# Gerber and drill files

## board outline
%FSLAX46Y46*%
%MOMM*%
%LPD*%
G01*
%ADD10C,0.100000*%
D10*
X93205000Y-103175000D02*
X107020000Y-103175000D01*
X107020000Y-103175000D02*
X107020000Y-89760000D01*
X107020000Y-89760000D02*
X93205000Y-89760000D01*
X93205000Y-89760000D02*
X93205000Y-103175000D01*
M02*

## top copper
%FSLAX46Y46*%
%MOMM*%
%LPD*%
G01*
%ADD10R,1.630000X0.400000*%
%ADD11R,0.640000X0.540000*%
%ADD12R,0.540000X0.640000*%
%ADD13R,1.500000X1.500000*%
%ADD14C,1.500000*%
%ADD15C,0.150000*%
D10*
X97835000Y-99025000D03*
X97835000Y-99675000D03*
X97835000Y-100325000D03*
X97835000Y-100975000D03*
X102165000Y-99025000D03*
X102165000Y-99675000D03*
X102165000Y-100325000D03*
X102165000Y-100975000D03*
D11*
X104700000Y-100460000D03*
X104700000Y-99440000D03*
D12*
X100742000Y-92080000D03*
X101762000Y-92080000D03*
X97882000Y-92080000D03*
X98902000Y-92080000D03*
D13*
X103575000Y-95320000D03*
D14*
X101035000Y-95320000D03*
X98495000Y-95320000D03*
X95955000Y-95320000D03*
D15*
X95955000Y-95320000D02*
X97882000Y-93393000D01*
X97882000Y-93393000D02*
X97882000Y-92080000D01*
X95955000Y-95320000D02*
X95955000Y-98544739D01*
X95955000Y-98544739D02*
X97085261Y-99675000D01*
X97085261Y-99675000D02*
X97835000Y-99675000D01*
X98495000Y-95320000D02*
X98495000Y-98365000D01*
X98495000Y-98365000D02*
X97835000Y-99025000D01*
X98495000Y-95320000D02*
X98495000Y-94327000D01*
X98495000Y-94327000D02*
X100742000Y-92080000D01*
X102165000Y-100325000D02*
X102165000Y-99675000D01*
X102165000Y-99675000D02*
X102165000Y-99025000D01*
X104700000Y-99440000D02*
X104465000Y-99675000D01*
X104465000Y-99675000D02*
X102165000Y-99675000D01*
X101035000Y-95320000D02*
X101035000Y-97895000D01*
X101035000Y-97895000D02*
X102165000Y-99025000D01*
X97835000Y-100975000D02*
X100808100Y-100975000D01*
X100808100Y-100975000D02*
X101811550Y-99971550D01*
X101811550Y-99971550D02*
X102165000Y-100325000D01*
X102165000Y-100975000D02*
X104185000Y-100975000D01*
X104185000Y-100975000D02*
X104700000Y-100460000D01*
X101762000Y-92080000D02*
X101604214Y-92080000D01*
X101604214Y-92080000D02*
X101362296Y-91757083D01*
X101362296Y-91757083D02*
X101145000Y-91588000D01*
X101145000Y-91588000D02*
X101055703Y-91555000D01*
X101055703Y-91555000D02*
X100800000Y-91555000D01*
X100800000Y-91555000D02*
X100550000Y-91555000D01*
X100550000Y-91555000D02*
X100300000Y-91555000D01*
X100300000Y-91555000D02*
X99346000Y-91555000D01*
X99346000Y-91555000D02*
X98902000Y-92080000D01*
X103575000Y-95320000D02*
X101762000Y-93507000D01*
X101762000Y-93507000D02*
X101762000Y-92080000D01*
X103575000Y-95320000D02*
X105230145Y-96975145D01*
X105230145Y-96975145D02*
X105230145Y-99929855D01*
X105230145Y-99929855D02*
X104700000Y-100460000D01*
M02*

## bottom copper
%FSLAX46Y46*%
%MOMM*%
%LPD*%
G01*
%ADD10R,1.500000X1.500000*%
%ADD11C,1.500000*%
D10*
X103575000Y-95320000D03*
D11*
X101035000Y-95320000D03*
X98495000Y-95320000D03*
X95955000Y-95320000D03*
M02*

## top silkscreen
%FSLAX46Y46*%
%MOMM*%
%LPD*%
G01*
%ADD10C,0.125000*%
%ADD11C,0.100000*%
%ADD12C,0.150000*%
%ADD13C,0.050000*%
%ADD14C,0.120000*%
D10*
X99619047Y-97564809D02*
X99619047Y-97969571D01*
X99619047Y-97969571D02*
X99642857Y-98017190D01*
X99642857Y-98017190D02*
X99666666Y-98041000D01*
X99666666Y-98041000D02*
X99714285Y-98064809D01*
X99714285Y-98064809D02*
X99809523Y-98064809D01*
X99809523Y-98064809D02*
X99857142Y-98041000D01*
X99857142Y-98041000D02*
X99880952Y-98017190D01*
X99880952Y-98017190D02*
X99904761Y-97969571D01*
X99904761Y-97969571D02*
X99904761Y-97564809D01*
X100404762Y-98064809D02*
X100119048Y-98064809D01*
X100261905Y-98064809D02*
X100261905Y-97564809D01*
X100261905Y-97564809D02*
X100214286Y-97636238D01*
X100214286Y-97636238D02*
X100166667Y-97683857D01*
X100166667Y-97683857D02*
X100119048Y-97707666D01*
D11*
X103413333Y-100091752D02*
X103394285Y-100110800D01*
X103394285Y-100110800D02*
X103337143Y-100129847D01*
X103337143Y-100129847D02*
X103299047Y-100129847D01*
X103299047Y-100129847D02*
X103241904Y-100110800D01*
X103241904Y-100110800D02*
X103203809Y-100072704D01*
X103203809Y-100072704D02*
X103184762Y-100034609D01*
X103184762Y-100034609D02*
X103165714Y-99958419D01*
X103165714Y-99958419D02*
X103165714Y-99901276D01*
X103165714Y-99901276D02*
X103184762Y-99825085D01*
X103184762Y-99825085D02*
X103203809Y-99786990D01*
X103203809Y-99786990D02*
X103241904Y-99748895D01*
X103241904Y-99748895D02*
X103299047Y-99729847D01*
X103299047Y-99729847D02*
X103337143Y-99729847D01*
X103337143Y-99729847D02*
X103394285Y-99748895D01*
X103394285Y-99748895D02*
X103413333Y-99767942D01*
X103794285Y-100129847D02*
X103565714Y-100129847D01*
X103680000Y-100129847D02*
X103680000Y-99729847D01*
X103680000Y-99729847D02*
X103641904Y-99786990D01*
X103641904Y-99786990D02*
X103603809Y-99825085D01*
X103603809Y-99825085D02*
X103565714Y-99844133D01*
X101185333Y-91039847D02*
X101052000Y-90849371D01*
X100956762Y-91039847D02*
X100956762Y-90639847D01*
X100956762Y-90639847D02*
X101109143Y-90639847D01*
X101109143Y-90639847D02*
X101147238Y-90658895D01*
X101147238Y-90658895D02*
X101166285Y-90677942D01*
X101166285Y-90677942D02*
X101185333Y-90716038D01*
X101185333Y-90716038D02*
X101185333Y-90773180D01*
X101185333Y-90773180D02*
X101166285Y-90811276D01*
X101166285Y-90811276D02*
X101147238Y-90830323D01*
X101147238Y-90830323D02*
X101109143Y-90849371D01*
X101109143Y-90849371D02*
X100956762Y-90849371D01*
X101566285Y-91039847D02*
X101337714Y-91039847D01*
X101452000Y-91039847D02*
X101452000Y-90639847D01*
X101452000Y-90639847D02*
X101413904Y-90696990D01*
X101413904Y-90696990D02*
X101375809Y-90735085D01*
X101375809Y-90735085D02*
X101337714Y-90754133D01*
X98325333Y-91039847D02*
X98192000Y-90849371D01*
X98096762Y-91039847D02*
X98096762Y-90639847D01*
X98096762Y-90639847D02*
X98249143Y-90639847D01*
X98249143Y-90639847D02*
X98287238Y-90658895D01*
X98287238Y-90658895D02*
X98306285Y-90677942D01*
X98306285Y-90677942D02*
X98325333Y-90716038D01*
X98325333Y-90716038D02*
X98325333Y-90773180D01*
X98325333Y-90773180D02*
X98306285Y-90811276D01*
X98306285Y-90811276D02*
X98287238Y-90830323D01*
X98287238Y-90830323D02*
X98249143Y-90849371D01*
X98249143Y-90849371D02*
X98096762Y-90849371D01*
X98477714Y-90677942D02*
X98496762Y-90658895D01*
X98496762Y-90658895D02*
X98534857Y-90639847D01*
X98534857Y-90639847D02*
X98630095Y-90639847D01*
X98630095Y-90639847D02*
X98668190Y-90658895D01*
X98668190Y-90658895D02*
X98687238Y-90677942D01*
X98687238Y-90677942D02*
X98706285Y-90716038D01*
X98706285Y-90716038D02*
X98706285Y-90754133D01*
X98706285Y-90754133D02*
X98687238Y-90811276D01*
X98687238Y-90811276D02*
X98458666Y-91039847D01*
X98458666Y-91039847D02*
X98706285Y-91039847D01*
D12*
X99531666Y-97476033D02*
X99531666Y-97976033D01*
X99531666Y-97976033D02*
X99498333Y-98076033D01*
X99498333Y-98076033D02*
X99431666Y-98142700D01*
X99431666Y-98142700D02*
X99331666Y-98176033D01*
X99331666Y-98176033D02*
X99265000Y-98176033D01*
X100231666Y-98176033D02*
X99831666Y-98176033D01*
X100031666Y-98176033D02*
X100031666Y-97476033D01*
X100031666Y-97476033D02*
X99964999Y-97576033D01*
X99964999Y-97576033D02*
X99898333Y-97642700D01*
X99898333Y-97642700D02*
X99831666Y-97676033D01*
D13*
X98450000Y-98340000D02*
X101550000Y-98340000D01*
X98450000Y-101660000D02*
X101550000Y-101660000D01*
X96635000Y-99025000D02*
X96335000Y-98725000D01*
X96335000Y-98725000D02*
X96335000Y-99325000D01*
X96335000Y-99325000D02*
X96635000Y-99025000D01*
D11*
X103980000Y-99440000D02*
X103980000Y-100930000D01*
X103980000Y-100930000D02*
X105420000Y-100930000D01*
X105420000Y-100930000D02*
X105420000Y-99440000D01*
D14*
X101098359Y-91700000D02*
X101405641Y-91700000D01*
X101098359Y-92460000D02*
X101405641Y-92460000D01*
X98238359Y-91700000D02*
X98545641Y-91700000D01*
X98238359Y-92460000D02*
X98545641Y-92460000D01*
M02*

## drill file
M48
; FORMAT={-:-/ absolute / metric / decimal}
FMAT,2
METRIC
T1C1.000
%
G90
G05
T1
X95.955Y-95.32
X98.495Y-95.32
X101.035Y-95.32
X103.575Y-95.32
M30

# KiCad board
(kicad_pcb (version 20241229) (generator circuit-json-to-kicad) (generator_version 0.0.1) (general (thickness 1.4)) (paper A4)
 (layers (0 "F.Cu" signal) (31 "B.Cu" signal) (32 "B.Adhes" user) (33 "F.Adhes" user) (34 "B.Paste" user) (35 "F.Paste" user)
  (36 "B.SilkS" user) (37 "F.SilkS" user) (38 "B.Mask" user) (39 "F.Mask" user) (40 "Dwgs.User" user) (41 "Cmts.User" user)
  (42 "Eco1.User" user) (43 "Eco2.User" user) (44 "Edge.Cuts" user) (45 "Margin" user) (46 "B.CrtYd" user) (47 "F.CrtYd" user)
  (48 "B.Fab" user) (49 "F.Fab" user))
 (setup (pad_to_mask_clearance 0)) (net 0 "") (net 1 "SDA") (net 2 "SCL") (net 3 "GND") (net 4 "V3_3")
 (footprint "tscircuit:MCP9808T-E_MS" (layer F.Cu) (at 100 100 0)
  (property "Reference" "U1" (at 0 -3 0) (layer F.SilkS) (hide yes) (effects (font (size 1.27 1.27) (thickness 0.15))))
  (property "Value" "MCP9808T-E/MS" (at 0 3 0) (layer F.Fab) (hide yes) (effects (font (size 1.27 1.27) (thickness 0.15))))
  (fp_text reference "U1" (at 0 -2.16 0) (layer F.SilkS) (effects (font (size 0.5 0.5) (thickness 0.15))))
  (fp_line (start -1.55 -1.66) (end 1.55 -1.66) (stroke (width 0.05) (type default)) (layer F.SilkS))
  (fp_line (start -1.55 1.66) (end 1.55 1.66) (stroke (width 0.05) (type default)) (layer F.SilkS))
  (fp_line (start -3.3649999999999998 -0.9750000000000001) (end -3.665 -1.2750000000000001) (stroke (width 0.05) (type default))
   (layer F.SilkS))
  (fp_line (start -3.665 -1.2750000000000001) (end -3.665 -0.675) (stroke (width 0.05) (type default)) (layer F.SilkS))
  (fp_line (start -3.665 -0.675) (end -3.3649999999999998 -0.9750000000000001) (stroke (width 0.05) (type default)) (layer F.SilkS))
  (pad "1" smd rect (at -2.165 -0.9750000000000001 0) (size 1.63 0.4) (layers F.Cu F.Paste F.Mask) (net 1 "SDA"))
  (pad "2" smd rect (at -2.165 -0.325 0) (size 1.63 0.4) (layers F.Cu F.Paste F.Mask) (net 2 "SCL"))
  (pad "3" smd rect (at -2.165 0.325 0) (size 1.63 0.4) (layers F.Cu F.Paste F.Mask))
  (pad "4" smd rect (at -2.165 0.9750000000000001 0) (size 1.63 0.4) (layers F.Cu F.Paste F.Mask) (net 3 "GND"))
  (pad "5" smd rect (at 2.165 -0.9750000000000001 0) (size 1.63 0.4) (layers F.Cu F.Paste F.Mask) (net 3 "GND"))
  (pad "6" smd rect (at 2.165 -0.325 0) (size 1.63 0.4) (layers F.Cu F.Paste F.Mask) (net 3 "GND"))
  (pad "7" smd rect (at 2.165 0.325 0) (size 1.63 0.4) (layers F.Cu F.Paste F.Mask) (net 3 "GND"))
  (pad "8" smd rect (at 2.165 0.9750000000000001 0) (size 1.63 0.4) (layers F.Cu F.Paste F.Mask) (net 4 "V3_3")))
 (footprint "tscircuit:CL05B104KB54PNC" (layer F.Cu) (at 104.7 99.95 90)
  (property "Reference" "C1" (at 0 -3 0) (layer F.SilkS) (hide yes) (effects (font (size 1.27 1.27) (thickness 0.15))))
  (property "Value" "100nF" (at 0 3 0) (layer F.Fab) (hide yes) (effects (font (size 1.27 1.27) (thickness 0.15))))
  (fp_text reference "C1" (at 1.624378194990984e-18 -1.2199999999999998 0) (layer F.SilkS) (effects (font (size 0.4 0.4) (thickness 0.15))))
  (fp_line (start 0.51 -0.7199999999999998) (end -0.98 -0.7200000000000001) (stroke (width 0.1) (type default)) (layer F.SilkS))
  (fp_line (start -0.98 -0.7200000000000001) (end -0.98 0.7199999999999999) (stroke (width 0.1) (type default)) (layer F.SilkS))
  (fp_line (start -0.98 0.7199999999999999) (end 0.51 0.7199999999999998) (stroke (width 0.1) (type default)) (layer F.SilkS))
  (pad "1" smd rect (at -0.51 0 0) (size 0.64 0.54) (layers F.Cu F.Paste F.Mask) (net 4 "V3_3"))
  (pad "2" smd rect (at 0.51 0 0) (size 0.64 0.54) (layers F.Cu F.Paste F.Mask) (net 3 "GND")))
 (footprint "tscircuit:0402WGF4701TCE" (layer F.Cu) (at 101.252 92.08 0)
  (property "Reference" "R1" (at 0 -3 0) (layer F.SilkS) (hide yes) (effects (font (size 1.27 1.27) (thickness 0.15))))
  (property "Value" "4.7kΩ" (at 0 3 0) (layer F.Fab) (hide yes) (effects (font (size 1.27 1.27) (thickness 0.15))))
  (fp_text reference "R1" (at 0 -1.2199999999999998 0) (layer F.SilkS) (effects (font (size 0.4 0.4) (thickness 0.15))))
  (fp_line (start -0.15364099999999992 -0.3799999999999999) (end 0.15364099999999992 -0.3799999999999999)
   (stroke (width 0.12) (type default)) (layer F.SilkS))
  (fp_line (start -0.15364099999999992 0.3799999999999999) (end 0.15364099999999992 0.3799999999999999) (stroke (width 0.12) (type default))
   (layer F.SilkS))
  (pad "1" smd rect (at -0.51 0 0) (size 0.54 0.64) (layers F.Cu F.Paste F.Mask) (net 1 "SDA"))
  (pad "2" smd rect (at 0.51 0 0) (size 0.54 0.64) (layers F.Cu F.Paste F.Mask) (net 4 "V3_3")))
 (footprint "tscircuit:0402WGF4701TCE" (layer F.Cu) (at 98.392 92.08 0)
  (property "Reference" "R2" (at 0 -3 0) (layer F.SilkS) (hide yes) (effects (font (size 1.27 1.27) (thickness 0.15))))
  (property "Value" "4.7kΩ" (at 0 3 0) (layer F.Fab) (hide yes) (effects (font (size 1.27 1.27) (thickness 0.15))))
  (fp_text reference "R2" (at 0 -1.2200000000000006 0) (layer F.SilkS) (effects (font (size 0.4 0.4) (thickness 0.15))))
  (fp_line (start -0.15364099999999992 -0.3800000000000008) (end 0.15364099999999992 -0.3800000000000008)
   (stroke (width 0.12) (type default)) (layer F.SilkS))
  (fp_line (start -0.15364099999999992 0.3799999999999999) (end 0.15364099999999992 0.3799999999999999) (stroke (width 0.12) (type default))
   (layer F.SilkS))
  (pad "1" smd rect (at -0.5099999999999998 0 0) (size 0.54 0.64) (layers F.Cu F.Paste F.Mask) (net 2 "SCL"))
  (pad "2" smd rect (at 0.51 0 0) (size 0.54 0.64) (layers F.Cu F.Paste F.Mask) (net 4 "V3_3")))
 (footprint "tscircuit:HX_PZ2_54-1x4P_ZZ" (layer F.Cu) (at 99.765 95.32 180)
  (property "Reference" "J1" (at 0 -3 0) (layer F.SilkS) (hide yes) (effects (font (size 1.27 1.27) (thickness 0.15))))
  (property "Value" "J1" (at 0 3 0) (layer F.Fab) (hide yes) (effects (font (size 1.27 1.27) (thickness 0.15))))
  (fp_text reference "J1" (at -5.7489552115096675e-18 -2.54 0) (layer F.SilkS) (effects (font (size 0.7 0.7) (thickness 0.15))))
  (pad "1" thru_hole rect (at -3.81 -4.215879892249837e-16 0) (size 1.5 1.5) (drill 1) (layers *.Cu *.Mask) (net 4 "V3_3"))
  (pad "2" thru_hole circle (at -1.27 1.5553014349171386e-16 0) (size 1.5 1.5) (drill 1) (layers *.Cu *.Mask) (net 3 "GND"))
  (pad "3" thru_hole circle (at 1.27 -1.5553014349171386e-16 0) (size 1.5 1.5) (drill 1) (layers *.Cu *.Mask) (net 1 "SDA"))
  (pad "4" thru_hole circle (at 3.8100000000000005 4.215879892249836e-16 0) (size 1.5 1.5) (drill 1) (layers *.Cu *.Mask) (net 2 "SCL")))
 (segment (start 95.955 95.32) (end 97.882 93.393) (width 0.15) (layer F.Cu) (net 2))
 (segment (start 97.882 93.393) (end 97.882 92.08) (width 0.15) (layer F.Cu) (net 2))
 (segment (start 95.955 95.32) (end 95.955 98.54473899217018) (width 0.15) (layer F.Cu) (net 2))
 (segment (start 95.955 98.54473899217018) (end 97.08526100782983 99.675) (width 0.15) (layer F.Cu) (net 2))
 (segment (start 97.08526100782983 99.675) (end 97.835 99.675) (width 0.15) (layer F.Cu) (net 2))
 (segment (start 98.495 95.32) (end 98.495 98.365) (width 0.15) (layer F.Cu) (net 1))
 (segment (start 98.495 98.365) (end 97.835 99.025) (width 0.15) (layer F.Cu) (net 1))
 (segment (start 98.495 95.32) (end 98.495 94.327) (width 0.15) (layer F.Cu) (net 1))
 (segment (start 98.495 94.327) (end 100.742 92.08) (width 0.15) (layer F.Cu) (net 1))
 (segment (start 102.165 100.325) (end 102.165 99.675) (width 0.15) (layer F.Cu) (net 3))
 (segment (start 102.165 99.675) (end 102.165 99.025) (width 0.15) (layer F.Cu) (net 3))
 (segment (start 104.7 99.44) (end 104.465 99.675) (width 0.15) (layer F.Cu) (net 3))
 (segment (start 104.465 99.675) (end 102.165 99.675) (width 0.15) (layer F.Cu) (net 3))
 (segment (start 101.035 95.32) (end 101.035 97.895) (width 0.15) (layer F.Cu) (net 3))
 (segment (start 101.035 97.895) (end 102.165 99.025) (width 0.15) (layer F.Cu) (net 3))
 (segment (start 97.835 100.975) (end 100.8081004428189 100.975) (width 0.15) (layer F.Cu) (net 3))
 (segment (start 100.8081004428189 100.975) (end 101.81155022140945 99.97155022140944) (width 0.15) (layer F.Cu) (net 3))
 (segment (start 101.81155022140945 99.97155022140944) (end 102.165 100.325) (width 0.15) (layer F.Cu) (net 3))
 (segment (start 102.165 100.975) (end 104.185 100.975) (width 0.15) (layer F.Cu) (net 4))
 (segment (start 104.185 100.975) (end 104.7 100.46) (width 0.15) (layer F.Cu) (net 4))
 (segment (start 101.762 92.08) (end 101.60421358827789 92.08) (width 0.15) (layer F.Cu) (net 4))
 (segment (start 101.60421358827789 92.08) (end 101.36229640972213 91.75708282144424) (width 0.15) (layer F.Cu) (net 4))
 (segment (start 101.36229640972213 91.75708282144424) (end 101.145 91.588) (width 0.15) (layer F.Cu) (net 4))
 (segment (start 101.145 91.588) (end 101.05570262747594 91.555) (width 0.15) (layer F.Cu) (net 4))
 (segment (start 101.05570262747594 91.555) (end 100.8 91.555) (width 0.15) (layer F.Cu) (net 4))
 (segment (start 100.8 91.555) (end 100.55 91.555) (width 0.15) (layer F.Cu) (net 4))
 (segment (start 100.55 91.555) (end 100.3 91.555) (width 0.15) (layer F.Cu) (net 4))
 (segment (start 100.3 91.555) (end 99.346 91.555) (width 0.15) (layer F.Cu) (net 4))
 (segment (start 99.346 91.555) (end 98.902 92.08) (width 0.15) (layer F.Cu) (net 4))
 (segment (start 103.575 95.32) (end 101.762 93.507) (width 0.15) (layer F.Cu) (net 4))
 (segment (start 101.762 93.507) (end 101.762 92.08) (width 0.15) (layer F.Cu) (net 4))
 (segment (start 103.575 95.32) (end 105.23014545291443 96.97514545291443) (width 0.15) (layer F.Cu) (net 4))
 (segment (start 105.23014545291443 96.97514545291443) (end 105.23014545291443 99.92985454708557) (width 0.15) (layer F.Cu) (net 4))
 (segment (start 105.23014545291443 99.92985454708557) (end 104.7 100.46) (width 0.15) (layer F.Cu) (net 4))
 (gr_line (start 93.205 103.175) (end 107.02 103.175) (width 0.1) (layer Edge.Cuts))
 (gr_line (start 107.02 103.175) (end 107.02 89.76) (width 0.1) (layer Edge.Cuts))
 (gr_line (start 107.02 89.76) (end 93.205 89.76) (width 0.1) (layer Edge.Cuts))
 (gr_line (start 93.205 89.76) (end 93.205 103.175) (width 0.1) (layer Edge.Cuts)))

